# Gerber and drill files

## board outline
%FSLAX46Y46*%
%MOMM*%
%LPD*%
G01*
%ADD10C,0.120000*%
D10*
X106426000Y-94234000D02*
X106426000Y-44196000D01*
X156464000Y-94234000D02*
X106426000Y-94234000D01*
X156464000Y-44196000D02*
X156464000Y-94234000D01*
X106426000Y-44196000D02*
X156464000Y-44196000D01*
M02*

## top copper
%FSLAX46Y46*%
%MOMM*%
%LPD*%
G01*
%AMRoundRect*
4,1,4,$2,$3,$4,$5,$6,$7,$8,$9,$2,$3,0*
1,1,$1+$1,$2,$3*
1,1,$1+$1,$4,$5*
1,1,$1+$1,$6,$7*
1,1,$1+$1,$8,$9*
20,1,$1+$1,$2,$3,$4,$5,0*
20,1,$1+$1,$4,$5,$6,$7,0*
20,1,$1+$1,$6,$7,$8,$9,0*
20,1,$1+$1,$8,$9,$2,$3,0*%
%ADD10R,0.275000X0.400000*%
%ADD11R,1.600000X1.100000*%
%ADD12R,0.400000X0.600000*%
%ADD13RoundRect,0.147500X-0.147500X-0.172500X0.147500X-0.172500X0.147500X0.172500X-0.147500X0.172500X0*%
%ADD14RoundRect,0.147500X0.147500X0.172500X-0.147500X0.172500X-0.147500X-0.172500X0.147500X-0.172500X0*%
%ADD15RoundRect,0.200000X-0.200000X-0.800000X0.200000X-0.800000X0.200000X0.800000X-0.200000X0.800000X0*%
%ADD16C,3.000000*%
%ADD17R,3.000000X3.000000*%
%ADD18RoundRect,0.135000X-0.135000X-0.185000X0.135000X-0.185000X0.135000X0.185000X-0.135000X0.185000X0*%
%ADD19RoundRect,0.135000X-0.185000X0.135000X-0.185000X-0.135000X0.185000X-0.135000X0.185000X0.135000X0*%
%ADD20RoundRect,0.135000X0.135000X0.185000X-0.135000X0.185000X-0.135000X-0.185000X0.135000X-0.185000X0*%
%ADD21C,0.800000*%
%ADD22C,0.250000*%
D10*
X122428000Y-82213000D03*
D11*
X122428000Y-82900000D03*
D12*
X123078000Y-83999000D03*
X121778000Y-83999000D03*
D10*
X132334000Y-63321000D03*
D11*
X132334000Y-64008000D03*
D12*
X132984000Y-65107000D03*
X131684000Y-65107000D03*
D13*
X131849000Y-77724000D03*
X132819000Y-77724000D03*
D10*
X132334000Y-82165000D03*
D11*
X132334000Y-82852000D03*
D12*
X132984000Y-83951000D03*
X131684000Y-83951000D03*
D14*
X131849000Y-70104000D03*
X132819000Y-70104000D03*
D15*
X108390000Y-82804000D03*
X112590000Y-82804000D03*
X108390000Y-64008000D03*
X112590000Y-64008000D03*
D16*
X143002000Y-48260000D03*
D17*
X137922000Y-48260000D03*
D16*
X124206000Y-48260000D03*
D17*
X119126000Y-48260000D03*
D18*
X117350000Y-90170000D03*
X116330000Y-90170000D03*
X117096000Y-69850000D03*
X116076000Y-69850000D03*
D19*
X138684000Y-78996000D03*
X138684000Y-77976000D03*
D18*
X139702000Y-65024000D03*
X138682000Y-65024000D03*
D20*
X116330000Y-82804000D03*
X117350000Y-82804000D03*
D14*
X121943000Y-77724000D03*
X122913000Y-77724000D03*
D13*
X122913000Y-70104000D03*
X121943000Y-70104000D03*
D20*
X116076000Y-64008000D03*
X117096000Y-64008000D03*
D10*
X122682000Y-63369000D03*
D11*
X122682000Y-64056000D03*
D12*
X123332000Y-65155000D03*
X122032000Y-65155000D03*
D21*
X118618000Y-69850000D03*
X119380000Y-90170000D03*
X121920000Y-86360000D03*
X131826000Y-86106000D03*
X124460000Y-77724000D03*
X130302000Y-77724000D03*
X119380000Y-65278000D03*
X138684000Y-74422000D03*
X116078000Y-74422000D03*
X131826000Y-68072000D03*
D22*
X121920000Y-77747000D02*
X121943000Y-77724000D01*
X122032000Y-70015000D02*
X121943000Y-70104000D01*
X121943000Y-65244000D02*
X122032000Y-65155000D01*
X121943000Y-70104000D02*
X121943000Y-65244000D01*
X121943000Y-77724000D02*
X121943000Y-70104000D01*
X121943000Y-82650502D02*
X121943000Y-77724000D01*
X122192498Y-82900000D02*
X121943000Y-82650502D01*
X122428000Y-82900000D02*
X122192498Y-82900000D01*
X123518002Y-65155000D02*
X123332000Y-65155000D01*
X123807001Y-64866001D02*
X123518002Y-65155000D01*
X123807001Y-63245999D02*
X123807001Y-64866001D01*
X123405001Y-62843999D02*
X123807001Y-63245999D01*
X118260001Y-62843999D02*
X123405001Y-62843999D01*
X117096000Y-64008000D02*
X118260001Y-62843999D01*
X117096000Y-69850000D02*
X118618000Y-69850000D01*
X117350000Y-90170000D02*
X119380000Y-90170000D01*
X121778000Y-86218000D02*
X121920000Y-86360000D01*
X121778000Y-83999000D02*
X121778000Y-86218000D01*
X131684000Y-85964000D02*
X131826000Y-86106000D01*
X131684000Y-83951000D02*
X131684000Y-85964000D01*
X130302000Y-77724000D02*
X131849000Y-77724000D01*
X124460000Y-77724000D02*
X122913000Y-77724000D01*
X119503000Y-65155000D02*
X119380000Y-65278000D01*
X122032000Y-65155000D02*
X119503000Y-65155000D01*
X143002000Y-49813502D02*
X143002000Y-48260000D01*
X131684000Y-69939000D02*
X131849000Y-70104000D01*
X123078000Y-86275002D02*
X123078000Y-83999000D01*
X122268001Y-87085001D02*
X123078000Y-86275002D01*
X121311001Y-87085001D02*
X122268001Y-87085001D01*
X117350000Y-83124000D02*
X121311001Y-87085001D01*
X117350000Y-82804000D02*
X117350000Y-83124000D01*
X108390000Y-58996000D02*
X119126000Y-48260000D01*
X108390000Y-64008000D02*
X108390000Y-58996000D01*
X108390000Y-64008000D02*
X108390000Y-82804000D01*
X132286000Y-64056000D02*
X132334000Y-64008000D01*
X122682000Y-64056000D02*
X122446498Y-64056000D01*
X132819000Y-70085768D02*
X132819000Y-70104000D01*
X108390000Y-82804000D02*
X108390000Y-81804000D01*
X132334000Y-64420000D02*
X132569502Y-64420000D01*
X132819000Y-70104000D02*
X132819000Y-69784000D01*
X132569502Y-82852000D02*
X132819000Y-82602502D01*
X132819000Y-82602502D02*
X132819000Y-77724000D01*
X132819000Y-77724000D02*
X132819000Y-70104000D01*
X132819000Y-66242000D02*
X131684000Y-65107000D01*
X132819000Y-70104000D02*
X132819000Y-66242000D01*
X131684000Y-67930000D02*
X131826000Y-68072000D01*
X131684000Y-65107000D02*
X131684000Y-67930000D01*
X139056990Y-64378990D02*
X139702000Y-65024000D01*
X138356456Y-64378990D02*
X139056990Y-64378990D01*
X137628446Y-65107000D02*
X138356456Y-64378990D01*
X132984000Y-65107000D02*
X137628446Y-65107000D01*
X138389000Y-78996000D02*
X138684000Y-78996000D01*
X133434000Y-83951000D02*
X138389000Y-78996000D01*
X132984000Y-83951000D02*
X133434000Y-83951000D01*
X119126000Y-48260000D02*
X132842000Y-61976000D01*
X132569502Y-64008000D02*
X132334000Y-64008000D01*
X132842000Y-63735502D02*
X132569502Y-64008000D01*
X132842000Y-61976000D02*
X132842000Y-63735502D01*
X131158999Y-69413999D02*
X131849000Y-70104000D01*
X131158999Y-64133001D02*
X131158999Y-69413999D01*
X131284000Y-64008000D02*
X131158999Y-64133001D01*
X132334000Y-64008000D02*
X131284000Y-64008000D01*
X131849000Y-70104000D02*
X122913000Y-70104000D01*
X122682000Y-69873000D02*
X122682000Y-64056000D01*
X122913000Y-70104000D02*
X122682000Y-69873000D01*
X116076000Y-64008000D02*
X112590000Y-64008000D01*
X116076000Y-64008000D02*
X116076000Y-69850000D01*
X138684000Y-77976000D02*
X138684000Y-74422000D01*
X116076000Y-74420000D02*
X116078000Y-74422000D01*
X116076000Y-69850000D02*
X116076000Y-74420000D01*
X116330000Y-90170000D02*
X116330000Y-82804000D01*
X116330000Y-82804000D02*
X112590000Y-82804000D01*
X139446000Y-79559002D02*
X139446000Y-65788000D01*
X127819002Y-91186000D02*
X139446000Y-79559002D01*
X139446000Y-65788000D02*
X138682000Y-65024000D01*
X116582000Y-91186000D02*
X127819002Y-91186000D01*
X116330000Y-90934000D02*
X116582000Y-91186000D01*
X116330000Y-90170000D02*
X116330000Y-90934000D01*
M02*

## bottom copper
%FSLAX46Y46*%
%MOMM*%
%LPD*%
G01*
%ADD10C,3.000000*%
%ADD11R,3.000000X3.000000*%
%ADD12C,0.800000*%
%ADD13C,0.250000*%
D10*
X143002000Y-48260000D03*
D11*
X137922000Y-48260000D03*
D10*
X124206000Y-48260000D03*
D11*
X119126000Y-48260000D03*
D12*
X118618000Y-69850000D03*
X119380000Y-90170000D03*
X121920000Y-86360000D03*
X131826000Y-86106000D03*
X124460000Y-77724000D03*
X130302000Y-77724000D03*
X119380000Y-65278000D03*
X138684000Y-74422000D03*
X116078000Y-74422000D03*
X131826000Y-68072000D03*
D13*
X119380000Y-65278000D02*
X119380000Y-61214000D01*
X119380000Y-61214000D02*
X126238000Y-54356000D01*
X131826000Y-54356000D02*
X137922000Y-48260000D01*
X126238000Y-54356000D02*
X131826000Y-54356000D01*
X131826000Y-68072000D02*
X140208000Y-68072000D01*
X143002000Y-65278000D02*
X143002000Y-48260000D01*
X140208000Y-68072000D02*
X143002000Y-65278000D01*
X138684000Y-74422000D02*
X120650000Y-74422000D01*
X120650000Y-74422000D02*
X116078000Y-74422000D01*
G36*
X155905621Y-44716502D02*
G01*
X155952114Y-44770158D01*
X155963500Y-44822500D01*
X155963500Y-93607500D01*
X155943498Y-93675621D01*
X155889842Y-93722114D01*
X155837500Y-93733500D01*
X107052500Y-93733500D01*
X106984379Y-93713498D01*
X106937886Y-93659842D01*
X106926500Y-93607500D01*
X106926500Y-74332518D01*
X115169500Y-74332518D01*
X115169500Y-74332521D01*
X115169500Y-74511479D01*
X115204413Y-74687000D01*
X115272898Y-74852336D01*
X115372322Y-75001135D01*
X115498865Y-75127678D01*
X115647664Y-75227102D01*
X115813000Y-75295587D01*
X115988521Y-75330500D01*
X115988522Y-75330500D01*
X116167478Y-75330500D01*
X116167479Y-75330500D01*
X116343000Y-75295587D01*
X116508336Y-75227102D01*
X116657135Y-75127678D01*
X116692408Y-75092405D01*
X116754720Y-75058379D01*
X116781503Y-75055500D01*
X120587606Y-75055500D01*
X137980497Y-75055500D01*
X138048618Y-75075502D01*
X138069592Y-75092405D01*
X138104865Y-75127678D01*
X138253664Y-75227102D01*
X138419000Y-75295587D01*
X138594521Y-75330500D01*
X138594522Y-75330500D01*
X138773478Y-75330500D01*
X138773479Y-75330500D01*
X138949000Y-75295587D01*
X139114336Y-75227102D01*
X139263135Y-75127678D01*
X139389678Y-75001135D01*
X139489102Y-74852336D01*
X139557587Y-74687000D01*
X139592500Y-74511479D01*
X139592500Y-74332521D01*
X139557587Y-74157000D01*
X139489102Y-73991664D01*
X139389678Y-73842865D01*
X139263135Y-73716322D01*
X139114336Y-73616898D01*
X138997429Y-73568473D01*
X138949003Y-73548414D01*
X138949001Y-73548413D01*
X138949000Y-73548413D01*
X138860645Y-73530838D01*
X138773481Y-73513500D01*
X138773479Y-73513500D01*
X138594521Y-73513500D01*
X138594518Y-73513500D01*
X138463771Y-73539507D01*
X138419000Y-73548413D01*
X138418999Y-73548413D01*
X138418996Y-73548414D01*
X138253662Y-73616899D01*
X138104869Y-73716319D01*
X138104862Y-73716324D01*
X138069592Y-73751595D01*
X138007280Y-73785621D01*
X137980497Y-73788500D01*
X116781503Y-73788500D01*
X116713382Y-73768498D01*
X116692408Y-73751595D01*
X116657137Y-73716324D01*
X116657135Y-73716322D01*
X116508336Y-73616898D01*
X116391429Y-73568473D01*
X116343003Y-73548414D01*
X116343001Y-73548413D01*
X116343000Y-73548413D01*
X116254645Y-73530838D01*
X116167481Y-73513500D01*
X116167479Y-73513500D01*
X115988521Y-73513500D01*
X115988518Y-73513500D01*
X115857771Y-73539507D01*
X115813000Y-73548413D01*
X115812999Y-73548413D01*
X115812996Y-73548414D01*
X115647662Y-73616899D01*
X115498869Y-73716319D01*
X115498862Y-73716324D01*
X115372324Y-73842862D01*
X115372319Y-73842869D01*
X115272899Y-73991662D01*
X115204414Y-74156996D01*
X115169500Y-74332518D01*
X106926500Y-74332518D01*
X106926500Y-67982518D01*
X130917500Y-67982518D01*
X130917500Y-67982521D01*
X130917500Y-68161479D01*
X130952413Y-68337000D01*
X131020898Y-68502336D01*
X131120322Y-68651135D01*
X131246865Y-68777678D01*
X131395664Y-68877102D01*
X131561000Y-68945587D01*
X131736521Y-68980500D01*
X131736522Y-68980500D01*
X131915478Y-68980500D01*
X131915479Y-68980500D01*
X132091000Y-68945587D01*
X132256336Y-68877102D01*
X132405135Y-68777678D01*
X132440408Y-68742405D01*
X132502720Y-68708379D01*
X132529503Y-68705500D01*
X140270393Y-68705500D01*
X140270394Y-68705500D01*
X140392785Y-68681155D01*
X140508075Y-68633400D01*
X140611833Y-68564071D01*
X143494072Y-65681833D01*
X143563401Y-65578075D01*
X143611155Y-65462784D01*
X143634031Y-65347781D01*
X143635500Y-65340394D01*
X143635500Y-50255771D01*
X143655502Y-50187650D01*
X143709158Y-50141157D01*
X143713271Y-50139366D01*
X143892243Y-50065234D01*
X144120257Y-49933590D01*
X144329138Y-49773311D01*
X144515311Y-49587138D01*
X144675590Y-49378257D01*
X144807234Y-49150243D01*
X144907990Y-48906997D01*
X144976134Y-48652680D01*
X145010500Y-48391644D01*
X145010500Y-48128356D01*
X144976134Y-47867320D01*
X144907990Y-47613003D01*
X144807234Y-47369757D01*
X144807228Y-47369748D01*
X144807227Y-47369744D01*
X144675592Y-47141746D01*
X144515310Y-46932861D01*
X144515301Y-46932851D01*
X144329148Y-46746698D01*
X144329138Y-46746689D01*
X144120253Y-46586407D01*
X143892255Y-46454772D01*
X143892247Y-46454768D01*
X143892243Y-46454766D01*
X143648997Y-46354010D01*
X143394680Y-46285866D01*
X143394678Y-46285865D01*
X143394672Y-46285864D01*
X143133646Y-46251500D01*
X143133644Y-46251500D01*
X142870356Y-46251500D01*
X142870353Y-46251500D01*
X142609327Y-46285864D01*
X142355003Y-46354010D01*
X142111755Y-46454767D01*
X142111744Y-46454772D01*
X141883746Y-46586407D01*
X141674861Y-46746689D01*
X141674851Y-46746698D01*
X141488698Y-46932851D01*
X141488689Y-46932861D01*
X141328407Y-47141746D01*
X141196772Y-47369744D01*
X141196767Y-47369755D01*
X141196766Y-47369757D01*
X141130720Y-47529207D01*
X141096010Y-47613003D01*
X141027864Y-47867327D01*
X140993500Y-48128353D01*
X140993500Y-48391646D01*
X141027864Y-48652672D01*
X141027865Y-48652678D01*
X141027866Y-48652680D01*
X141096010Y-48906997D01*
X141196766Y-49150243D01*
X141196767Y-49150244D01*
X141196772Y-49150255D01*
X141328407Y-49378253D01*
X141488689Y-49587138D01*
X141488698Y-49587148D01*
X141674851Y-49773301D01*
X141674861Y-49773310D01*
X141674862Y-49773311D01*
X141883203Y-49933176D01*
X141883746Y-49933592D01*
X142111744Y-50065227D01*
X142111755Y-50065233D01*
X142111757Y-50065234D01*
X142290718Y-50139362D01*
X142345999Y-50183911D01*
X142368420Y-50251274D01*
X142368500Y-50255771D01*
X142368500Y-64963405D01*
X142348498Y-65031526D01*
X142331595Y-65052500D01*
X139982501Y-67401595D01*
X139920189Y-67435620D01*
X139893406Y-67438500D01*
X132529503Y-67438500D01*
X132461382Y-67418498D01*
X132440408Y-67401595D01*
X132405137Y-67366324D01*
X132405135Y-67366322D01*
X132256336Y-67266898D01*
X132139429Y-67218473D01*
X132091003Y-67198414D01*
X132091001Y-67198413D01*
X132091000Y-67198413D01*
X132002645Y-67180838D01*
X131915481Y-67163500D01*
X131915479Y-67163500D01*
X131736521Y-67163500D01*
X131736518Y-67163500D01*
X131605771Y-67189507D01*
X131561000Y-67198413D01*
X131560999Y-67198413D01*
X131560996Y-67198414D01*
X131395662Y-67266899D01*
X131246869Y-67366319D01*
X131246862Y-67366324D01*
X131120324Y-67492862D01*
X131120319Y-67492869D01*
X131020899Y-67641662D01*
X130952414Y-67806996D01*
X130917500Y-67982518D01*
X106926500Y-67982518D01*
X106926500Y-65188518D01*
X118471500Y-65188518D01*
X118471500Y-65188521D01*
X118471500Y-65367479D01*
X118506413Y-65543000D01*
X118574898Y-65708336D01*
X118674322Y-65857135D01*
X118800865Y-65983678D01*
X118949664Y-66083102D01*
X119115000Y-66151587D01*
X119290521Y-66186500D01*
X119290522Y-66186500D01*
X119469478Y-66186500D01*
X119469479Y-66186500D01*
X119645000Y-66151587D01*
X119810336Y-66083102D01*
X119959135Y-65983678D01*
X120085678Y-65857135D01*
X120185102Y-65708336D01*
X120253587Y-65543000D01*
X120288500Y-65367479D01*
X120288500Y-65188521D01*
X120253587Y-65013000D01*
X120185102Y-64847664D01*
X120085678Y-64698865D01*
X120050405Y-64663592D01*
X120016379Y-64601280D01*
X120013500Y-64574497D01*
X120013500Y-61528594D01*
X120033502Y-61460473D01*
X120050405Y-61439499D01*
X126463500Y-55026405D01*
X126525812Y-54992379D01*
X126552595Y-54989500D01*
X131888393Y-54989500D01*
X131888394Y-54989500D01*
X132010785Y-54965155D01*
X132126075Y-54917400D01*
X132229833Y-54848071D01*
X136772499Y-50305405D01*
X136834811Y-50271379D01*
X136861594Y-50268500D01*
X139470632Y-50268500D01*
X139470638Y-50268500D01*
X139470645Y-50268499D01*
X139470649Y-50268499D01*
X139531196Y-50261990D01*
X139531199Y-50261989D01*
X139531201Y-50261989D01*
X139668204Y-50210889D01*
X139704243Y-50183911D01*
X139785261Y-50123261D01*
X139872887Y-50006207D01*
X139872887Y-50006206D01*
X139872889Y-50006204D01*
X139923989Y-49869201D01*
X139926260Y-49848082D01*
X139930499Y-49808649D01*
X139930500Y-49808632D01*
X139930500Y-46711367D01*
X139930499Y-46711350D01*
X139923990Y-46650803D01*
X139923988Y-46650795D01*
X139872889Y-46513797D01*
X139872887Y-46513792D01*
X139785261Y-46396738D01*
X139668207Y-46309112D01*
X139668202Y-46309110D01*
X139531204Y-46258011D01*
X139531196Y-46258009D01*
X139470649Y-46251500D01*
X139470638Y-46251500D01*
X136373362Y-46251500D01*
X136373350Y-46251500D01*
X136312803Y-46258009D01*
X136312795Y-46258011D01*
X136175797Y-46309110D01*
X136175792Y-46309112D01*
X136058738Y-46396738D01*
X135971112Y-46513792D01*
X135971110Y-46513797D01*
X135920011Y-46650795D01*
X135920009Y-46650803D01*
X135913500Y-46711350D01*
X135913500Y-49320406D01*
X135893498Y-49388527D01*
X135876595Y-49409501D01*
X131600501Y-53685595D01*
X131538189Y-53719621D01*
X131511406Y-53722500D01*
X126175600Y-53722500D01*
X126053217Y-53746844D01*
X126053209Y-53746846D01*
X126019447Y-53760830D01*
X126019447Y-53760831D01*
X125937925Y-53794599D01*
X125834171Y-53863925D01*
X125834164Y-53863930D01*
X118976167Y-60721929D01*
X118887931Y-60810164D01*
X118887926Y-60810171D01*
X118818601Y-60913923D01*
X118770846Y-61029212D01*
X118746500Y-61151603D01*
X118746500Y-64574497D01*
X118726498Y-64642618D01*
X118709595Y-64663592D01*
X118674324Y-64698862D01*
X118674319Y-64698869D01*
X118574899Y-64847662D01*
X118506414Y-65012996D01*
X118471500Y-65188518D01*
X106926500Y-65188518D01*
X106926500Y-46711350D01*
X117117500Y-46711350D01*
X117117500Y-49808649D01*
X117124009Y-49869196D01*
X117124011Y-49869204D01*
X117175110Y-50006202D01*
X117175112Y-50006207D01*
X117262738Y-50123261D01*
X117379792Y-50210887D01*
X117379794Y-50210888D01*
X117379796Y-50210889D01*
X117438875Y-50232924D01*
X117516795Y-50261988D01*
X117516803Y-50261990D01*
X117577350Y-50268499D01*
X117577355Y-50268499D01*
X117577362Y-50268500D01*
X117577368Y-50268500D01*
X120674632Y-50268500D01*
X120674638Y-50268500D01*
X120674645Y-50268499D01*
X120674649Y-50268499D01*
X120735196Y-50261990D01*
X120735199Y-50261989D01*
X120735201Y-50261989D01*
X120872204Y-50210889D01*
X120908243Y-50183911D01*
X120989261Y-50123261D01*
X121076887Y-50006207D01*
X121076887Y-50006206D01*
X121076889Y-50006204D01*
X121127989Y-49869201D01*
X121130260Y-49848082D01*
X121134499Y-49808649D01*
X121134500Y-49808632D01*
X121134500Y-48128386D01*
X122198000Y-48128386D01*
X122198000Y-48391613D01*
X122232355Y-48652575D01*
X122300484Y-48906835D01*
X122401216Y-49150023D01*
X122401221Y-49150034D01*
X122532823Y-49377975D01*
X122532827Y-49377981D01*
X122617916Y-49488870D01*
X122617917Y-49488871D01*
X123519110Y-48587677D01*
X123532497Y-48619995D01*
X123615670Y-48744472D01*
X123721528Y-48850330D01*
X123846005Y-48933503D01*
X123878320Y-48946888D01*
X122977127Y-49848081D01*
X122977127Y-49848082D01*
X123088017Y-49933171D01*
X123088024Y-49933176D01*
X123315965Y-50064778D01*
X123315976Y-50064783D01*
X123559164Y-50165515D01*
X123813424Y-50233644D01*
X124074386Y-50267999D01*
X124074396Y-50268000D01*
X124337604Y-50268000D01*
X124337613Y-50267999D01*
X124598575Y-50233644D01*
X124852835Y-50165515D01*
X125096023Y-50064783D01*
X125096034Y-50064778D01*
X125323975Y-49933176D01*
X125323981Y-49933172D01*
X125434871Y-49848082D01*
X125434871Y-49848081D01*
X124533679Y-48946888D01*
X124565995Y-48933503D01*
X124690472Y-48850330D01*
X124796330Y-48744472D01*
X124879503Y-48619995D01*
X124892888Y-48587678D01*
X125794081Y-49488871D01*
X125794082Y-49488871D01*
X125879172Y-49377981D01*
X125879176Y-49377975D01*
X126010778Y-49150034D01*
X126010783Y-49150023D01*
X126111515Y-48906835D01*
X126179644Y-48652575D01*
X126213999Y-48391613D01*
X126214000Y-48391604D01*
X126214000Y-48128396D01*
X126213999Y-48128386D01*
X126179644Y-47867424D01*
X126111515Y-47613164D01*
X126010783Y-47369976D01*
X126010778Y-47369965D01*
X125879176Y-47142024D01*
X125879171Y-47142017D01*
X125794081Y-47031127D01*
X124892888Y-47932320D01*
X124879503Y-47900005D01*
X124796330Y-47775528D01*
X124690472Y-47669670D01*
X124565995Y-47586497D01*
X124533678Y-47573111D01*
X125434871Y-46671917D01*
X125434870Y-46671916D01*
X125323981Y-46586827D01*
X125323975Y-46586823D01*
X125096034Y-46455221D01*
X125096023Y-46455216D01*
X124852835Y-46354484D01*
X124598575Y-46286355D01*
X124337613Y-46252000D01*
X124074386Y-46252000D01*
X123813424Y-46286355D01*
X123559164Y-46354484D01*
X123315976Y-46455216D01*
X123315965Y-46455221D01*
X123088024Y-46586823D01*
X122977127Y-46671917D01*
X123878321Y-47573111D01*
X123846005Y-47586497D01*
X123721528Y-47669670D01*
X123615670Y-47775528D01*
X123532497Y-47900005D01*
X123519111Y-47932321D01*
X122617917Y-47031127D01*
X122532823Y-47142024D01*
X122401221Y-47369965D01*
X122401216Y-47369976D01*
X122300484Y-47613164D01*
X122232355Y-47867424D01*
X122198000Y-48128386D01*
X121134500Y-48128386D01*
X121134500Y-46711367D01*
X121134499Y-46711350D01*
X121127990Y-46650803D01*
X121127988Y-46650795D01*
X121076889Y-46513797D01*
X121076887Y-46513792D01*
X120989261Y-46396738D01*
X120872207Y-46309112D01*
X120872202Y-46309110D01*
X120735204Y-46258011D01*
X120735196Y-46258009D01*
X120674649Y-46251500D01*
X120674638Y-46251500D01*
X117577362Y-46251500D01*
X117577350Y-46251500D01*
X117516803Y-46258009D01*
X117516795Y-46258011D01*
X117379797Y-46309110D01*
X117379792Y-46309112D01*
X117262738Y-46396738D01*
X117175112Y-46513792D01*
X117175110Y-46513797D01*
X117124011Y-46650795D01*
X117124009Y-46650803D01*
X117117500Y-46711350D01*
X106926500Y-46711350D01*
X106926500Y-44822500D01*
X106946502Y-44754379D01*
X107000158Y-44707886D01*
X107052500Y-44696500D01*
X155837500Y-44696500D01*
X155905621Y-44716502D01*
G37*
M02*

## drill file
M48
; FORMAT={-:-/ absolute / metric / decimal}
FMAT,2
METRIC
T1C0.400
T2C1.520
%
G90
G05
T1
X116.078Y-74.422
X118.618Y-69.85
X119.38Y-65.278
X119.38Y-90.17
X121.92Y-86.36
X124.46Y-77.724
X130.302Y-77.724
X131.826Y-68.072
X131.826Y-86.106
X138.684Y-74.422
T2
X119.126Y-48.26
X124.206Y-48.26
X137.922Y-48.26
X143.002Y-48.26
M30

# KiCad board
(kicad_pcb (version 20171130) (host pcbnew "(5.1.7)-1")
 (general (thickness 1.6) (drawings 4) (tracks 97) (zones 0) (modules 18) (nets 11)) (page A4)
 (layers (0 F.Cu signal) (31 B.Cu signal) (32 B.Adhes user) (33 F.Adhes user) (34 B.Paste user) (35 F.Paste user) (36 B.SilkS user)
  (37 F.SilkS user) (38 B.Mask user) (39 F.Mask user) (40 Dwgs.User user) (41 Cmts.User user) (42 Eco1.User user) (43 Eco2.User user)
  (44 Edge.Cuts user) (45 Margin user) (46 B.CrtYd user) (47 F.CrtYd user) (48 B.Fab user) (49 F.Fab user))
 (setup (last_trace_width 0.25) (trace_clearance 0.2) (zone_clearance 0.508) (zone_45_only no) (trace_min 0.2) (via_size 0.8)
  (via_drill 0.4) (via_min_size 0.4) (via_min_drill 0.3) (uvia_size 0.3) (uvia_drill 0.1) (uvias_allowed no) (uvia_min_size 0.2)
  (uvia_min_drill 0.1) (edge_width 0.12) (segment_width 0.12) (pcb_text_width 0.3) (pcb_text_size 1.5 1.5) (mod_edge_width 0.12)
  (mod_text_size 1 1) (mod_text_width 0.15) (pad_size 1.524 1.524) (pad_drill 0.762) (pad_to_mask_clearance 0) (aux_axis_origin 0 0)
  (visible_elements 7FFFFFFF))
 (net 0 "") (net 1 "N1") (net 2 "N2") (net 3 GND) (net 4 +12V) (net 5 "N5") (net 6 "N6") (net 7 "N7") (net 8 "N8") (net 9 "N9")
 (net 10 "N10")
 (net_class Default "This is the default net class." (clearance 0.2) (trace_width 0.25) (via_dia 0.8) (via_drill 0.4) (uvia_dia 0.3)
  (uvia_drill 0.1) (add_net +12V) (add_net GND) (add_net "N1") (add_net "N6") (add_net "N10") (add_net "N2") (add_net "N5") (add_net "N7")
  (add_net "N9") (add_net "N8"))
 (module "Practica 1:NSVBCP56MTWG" (layer F.Cu) (at 122.428 83.106)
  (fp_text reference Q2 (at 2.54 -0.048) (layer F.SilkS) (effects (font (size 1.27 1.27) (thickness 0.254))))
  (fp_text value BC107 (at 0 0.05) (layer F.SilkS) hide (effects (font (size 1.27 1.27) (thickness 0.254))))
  (pad 4 smd rect (at 0 -0.893) (size 0.275 0.4) (layers F.Cu F.Paste F.Mask))
  (pad 3 smd rect (at 0 -0.206 90) (size 1.1 1.6) (layers F.Cu F.Paste F.Mask) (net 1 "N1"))
  (pad 2 smd rect (at 0.65 0.893) (size 0.4 0.6) (layers F.Cu F.Paste F.Mask) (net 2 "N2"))
  (pad 1 smd rect (at -0.65 0.893) (size 0.4 0.6) (layers F.Cu F.Paste F.Mask) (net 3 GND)))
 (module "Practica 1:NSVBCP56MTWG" (layer F.Cu) (at 132.334 64.214)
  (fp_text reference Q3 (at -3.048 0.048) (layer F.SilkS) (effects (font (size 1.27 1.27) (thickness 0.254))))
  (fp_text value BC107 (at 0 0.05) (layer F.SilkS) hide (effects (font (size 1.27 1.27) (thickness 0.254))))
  (pad 4 smd rect (at 0 -0.893) (size 0.275 0.4) (layers F.Cu F.Paste F.Mask))
  (pad 3 smd rect (at 0 -0.206 90) (size 1.1 1.6) (layers F.Cu F.Paste F.Mask) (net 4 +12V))
  (pad 2 smd rect (at 0.65 0.893) (size 0.4 0.6) (layers F.Cu F.Paste F.Mask) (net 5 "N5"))
  (pad 1 smd rect (at -0.65 0.893) (size 0.4 0.6) (layers F.Cu F.Paste F.Mask) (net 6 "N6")))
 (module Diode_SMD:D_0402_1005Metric (layer F.Cu) (at 132.334 77.724)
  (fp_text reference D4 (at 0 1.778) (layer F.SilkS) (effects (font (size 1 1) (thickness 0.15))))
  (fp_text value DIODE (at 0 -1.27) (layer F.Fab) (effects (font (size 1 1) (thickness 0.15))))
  (pad 1 smd roundrect (at -0.485 0) (size 0.59 0.64) (layers F.Cu F.Paste F.Mask) (roundrect_rratio 0.25) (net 3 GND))
  (pad 2 smd roundrect (at 0.485 0) (size 0.59 0.64) (layers F.Cu F.Paste F.Mask) (roundrect_rratio 0.25) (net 6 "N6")))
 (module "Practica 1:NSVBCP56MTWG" (layer F.Cu) (at 132.334 83.058)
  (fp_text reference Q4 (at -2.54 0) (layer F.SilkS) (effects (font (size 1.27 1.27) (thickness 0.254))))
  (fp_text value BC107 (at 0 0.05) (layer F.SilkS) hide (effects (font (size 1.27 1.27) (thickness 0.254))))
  (pad 4 smd rect (at 0 -0.893) (size 0.275 0.4) (layers F.Cu F.Paste F.Mask))
  (pad 3 smd rect (at 0 -0.206 90) (size 1.1 1.6) (layers F.Cu F.Paste F.Mask) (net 6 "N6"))
  (pad 2 smd rect (at 0.65 0.893) (size 0.4 0.6) (layers F.Cu F.Paste F.Mask) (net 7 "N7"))
  (pad 1 smd rect (at -0.65 0.893) (size 0.4 0.6) (layers F.Cu F.Paste F.Mask) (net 3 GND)))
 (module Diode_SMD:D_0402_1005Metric (layer F.Cu) (at 132.334 70.104 180)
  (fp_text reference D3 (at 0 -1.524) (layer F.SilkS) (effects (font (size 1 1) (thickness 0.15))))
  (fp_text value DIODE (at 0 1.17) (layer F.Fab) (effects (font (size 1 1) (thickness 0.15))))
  (pad 2 smd roundrect (at 0.485 0 180) (size 0.59 0.64) (layers F.Cu F.Paste F.Mask) (roundrect_rratio 0.25) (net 4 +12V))
  (pad 1 smd roundrect (at -0.485 0 180) (size 0.59 0.64) (layers F.Cu F.Paste F.Mask) (roundrect_rratio 0.25) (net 6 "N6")))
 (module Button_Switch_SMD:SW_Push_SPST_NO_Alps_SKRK (layer F.Cu) (at 110.49 82.804)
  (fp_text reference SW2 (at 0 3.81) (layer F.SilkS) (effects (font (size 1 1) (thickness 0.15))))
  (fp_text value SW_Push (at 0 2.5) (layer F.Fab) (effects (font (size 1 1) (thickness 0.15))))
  (pad 1 smd roundrect (at -2.1 0) (size 0.8 2) (layers F.Cu F.Paste F.Mask) (roundrect_rratio 0.25) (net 4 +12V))
  (pad 2 smd roundrect (at 2.1 0) (size 0.8 2) (layers F.Cu F.Paste F.Mask) (roundrect_rratio 0.25) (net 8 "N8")))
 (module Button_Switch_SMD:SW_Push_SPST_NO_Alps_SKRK (layer F.Cu) (at 110.49 64.008)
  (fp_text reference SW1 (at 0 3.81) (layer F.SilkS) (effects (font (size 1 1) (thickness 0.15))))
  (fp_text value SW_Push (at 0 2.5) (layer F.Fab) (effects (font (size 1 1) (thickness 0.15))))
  (pad 1 smd roundrect (at -2.1 0) (size 0.8 2) (layers F.Cu F.Paste F.Mask) (roundrect_rratio 0.25) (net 4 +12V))
  (pad 2 smd roundrect (at 2.1 0) (size 0.8 2) (layers F.Cu F.Paste F.Mask) (roundrect_rratio 0.25) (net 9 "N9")))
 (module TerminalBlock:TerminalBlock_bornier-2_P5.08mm (layer F.Cu) (at 137.922 48.26)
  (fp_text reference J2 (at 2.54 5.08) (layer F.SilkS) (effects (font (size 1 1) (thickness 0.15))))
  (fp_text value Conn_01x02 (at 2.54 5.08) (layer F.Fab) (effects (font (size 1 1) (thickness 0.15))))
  (pad 2 thru_hole circle (at 5.08 0) (size 3 3) (drill 1.52) (layers *.Cu *.Mask) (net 6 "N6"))
  (pad 1 thru_hole rect (at 0 0) (size 3 3) (drill 1.52) (layers *.Cu *.Mask) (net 1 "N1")))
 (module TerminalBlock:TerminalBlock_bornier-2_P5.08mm (layer F.Cu) (at 119.126 48.26)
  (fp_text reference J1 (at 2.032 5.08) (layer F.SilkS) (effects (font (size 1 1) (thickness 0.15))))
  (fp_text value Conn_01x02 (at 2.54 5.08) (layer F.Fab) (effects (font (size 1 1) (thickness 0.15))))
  (pad 2 thru_hole circle (at 5.08 0) (size 3 3) (drill 1.52) (layers *.Cu *.Mask) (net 3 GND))
  (pad 1 thru_hole rect (at 0 0) (size 3 3) (drill 1.52) (layers *.Cu *.Mask) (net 4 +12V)))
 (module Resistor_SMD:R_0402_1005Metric (layer F.Cu) (at 116.84 90.17)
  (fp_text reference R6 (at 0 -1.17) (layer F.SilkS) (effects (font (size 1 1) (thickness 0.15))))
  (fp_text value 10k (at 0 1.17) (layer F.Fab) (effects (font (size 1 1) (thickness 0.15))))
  (pad 2 smd roundrect (at 0.51 0) (size 0.54 0.64) (layers F.Cu F.Paste F.Mask) (roundrect_rratio 0.25) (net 3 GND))
  (pad 1 smd roundrect (at -0.51 0) (size 0.54 0.64) (layers F.Cu F.Paste F.Mask) (roundrect_rratio 0.25) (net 8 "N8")))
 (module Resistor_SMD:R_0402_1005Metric (layer F.Cu) (at 116.586 69.85)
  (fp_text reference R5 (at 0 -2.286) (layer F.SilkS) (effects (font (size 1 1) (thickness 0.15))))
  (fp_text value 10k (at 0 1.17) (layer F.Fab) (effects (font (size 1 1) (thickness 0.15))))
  (pad 2 smd roundrect (at 0.51 0) (size 0.54 0.64) (layers F.Cu F.Paste F.Mask) (roundrect_rratio 0.25) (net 3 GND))
  (pad 1 smd roundrect (at -0.51 0) (size 0.54 0.64) (layers F.Cu F.Paste F.Mask) (roundrect_rratio 0.25) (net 9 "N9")))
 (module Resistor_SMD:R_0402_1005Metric (layer F.Cu) (at 138.684 78.486 270)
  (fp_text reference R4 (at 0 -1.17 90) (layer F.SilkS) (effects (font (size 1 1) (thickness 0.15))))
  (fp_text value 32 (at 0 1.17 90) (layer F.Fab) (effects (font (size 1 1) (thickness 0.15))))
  (pad 2 smd roundrect (at 0.51 0 270) (size 0.54 0.64) (layers F.Cu F.Paste F.Mask) (roundrect_rratio 0.25) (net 7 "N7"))
  (pad 1 smd roundrect (at -0.51 0 270) (size 0.54 0.64) (layers F.Cu F.Paste F.Mask) (roundrect_rratio 0.25) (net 9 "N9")))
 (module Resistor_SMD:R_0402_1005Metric (layer F.Cu) (at 139.192 65.024)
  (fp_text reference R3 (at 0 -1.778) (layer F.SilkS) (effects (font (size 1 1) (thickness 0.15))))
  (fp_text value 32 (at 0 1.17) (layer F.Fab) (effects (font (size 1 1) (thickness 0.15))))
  (pad 2 smd roundrect (at 0.51 0) (size 0.54 0.64) (layers F.Cu F.Paste F.Mask) (roundrect_rratio 0.25) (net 5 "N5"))
  (pad 1 smd roundrect (at -0.51 0) (size 0.54 0.64) (layers F.Cu F.Paste F.Mask) (roundrect_rratio 0.25) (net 8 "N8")))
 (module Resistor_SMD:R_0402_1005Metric (layer F.Cu) (at 116.84 82.804 180)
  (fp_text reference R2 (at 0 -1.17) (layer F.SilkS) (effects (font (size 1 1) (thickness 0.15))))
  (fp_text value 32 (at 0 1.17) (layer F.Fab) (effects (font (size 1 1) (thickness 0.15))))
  (pad 2 smd roundrect (at 0.51 0 180) (size 0.54 0.64) (layers F.Cu F.Paste F.Mask) (roundrect_rratio 0.25) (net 8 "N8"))
  (pad 1 smd roundrect (at -0.51 0 180) (size 0.54 0.64) (layers F.Cu F.Paste F.Mask) (roundrect_rratio 0.25) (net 2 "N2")))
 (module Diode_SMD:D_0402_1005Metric (layer F.Cu) (at 122.428 77.724 180)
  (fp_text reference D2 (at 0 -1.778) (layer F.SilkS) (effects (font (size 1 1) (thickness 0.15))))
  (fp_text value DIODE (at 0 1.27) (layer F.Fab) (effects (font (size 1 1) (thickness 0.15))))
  (pad 2 smd roundrect (at 0.485 0 180) (size 0.59 0.64) (layers F.Cu F.Paste F.Mask) (roundrect_rratio 0.25) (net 1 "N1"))
  (pad 1 smd roundrect (at -0.485 0 180) (size 0.59 0.64) (layers F.Cu F.Paste F.Mask) (roundrect_rratio 0.25) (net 3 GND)))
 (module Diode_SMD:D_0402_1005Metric (layer F.Cu) (at 122.428 70.104)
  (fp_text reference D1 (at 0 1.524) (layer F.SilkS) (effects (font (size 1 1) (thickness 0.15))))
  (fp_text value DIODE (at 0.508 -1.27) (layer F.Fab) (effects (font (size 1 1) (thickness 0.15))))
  (pad 2 smd roundrect (at 0.485 0) (size 0.59 0.64) (layers F.Cu F.Paste F.Mask) (roundrect_rratio 0.25) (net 4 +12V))
  (pad 1 smd roundrect (at -0.485 0) (size 0.59 0.64) (layers F.Cu F.Paste F.Mask) (roundrect_rratio 0.25) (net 1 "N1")))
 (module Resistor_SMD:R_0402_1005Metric (layer F.Cu) (at 116.586 64.008 180)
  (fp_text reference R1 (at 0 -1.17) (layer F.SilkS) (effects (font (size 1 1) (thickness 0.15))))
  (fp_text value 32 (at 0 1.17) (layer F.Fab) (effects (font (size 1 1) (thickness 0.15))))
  (pad 2 smd roundrect (at 0.51 0 180) (size 0.54 0.64) (layers F.Cu F.Paste F.Mask) (roundrect_rratio 0.25) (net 9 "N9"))
  (pad 1 smd roundrect (at -0.51 0 180) (size 0.54 0.64) (layers F.Cu F.Paste F.Mask) (roundrect_rratio 0.25) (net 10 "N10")))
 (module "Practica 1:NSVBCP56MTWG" (layer F.Cu) (at 122.682 64.262)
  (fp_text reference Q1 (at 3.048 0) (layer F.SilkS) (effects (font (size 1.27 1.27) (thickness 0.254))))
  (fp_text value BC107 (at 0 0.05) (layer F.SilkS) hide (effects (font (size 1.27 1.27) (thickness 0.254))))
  (pad 4 smd rect (at 0 -0.893) (size 0.275 0.4) (layers F.Cu F.Paste F.Mask))
  (pad 3 smd rect (at 0 -0.206 90) (size 1.1 1.6) (layers F.Cu F.Paste F.Mask) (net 4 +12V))
  (pad 2 smd rect (at 0.65 0.893) (size 0.4 0.6) (layers F.Cu F.Paste F.Mask) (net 10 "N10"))
  (pad 1 smd rect (at -0.65 0.893) (size 0.4 0.6) (layers F.Cu F.Paste F.Mask) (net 1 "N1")))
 (gr_line (start 106.426 94.234) (end 106.426 44.196) (layer Edge.Cuts) (width 0.12))
 (gr_line (start 156.464 94.234) (end 106.426 94.234) (layer Edge.Cuts) (width 0.12))
 (gr_line (start 156.464 44.196) (end 156.464 94.234) (layer Edge.Cuts) (width 0.12))
 (gr_line (start 106.426 44.196) (end 156.464 44.196) (layer Edge.Cuts) (width 0.12))
 (via (at 118.618 69.85) (size 0.8) (drill 0.4) (layers F.Cu B.Cu) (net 3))
 (segment (start 121.92 77.747) (end 121.943 77.724) (width 0.25) (layer F.Cu) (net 1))
 (segment (start 122.032 70.015) (end 121.943 70.104) (width 0.25) (layer F.Cu) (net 1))
 (segment (start 121.943 65.244) (end 122.032 65.155) (width 0.25) (layer F.Cu) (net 1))
 (segment (start 121.943 70.104) (end 121.943 65.244) (width 0.25) (layer F.Cu) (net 1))
 (segment (start 121.943 77.724) (end 121.943 70.104) (width 0.25) (layer F.Cu) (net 1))
 (segment (start 121.943 82.650502) (end 121.943 77.724) (width 0.25) (layer F.Cu) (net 1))
 (segment (start 122.192498 82.9) (end 121.943 82.650502) (width 0.25) (layer F.Cu) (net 1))
 (segment (start 122.428 82.9) (end 122.192498 82.9) (width 0.25) (layer F.Cu) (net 1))
 (segment (start 123.518002 65.155) (end 123.332 65.155) (width 0.25) (layer F.Cu) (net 10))
 (segment (start 123.807001 64.866001) (end 123.518002 65.155) (width 0.25) (layer F.Cu) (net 10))
 (segment (start 123.807001 63.245999) (end 123.807001 64.866001) (width 0.25) (layer F.Cu) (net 10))
 (segment (start 123.405001 62.843999) (end 123.807001 63.245999) (width 0.25) (layer F.Cu) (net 10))
 (segment (start 118.260001 62.843999) (end 123.405001 62.843999) (width 0.25) (layer F.Cu) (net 10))
 (segment (start 117.096 64.008) (end 118.260001 62.843999) (width 0.25) (layer F.Cu) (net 10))
 (segment (start 117.096 69.85) (end 118.618 69.85) (width 0.25) (layer F.Cu) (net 3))
 (via (at 119.38 90.17) (size 0.8) (drill 0.4) (layers F.Cu B.Cu) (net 3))
 (segment (start 117.35 90.17) (end 119.38 90.17) (width 0.25) (layer F.Cu) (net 3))
 (via (at 121.92 86.36) (size 0.8) (drill 0.4) (layers F.Cu B.Cu) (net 3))
 (segment (start 121.778 86.218) (end 121.92 86.36) (width 0.25) (layer F.Cu) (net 3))
 (segment (start 121.778 83.999) (end 121.778 86.218) (width 0.25) (layer F.Cu) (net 3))
 (via (at 131.826 86.106) (size 0.8) (drill 0.4) (layers F.Cu B.Cu) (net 3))
 (segment (start 131.684 85.964) (end 131.826 86.106) (width 0.25) (layer F.Cu) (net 3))
 (segment (start 131.684 83.951) (end 131.684 85.964) (width 0.25) (layer F.Cu) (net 3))
 (via (at 124.46 77.724) (size 0.8) (drill 0.4) (layers F.Cu B.Cu) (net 3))
 (via (at 130.302 77.724) (size 0.8) (drill 0.4) (layers F.Cu B.Cu) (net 3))
 (segment (start 130.302 77.724) (end 131.849 77.724) (width 0.25) (layer F.Cu) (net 3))
 (segment (start 124.46 77.724) (end 122.913 77.724) (width 0.25) (layer F.Cu) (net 3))
 (via (at 119.38 65.278) (size 0.8) (drill 0.4) (layers F.Cu B.Cu) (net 1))
 (segment (start 119.503 65.155) (end 119.38 65.278) (width 0.25) (layer F.Cu) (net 1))
 (segment (start 122.032 65.155) (end 119.503 65.155) (width 0.25) (layer F.Cu) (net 1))
 (segment (start 119.38 65.278) (end 119.38 61.214) (width 0.25) (layer B.Cu) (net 1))
 (segment (start 119.38 61.214) (end 126.238 54.356) (width 0.25) (layer B.Cu) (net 1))
 (segment (start 131.826 54.356) (end 137.922 48.26) (width 0.25) (layer B.Cu) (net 1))
 (segment (start 126.238 54.356) (end 131.826 54.356) (width 0.25) (layer B.Cu) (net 1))
 (via (at 138.684 74.422) (size 0.8) (drill 0.4) (layers F.Cu B.Cu) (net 9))
 (via (at 116.078 74.422) (size 0.8) (drill 0.4) (layers F.Cu B.Cu) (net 9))
 (via (at 131.826 68.072) (size 0.8) (drill 0.4) (layers F.Cu B.Cu) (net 6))
 (segment (start 143.002 49.813502) (end 143.002 48.26) (width 0.25) (layer F.Cu) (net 6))
 (segment (start 131.684 69.939) (end 131.849 70.104) (width 0.25) (layer F.Cu) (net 4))
 (segment (start 123.078 86.275002) (end 123.078 83.999) (width 0.25) (layer F.Cu) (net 2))
 (segment (start 122.268001 87.085001) (end 123.078 86.275002) (width 0.25) (layer F.Cu) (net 2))
 (segment (start 121.311001 87.085001) (end 122.268001 87.085001) (width 0.25) (layer F.Cu) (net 2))
 (segment (start 117.35 83.124) (end 121.311001 87.085001) (width 0.25) (layer F.Cu) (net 2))
 (segment (start 117.35 82.804) (end 117.35 83.124) (width 0.25) (layer F.Cu) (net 2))
 (segment (start 108.39 58.996) (end 119.126 48.26) (width 0.25) (layer F.Cu) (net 4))
 (segment (start 108.39 64.008) (end 108.39 58.996) (width 0.25) (layer F.Cu) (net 4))
 (segment (start 108.39 64.008) (end 108.39 82.804) (width 0.25) (layer F.Cu) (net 4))
 (segment (start 132.286 64.056) (end 132.334 64.008) (width 0.25) (layer F.Cu) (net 4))
 (segment (start 122.682 64.056) (end 122.446498 64.056) (width 0.25) (layer F.Cu) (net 4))
 (segment (start 132.819 70.085768) (end 132.819 70.104) (width 0.25) (layer F.Cu) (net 6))
 (segment (start 108.39 82.804) (end 108.39 81.804) (width 0.25) (layer F.Cu) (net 4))
 (segment (start 132.334 64.42) (end 132.569502 64.42) (width 0.25) (layer F.Cu) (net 4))
 (segment (start 132.819 70.104) (end 132.819 69.784) (width 0.25) (layer F.Cu) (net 6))
 (segment (start 132.569502 82.852) (end 132.819 82.602502) (width 0.25) (layer F.Cu) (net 6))
 (segment (start 132.819 82.602502) (end 132.819 77.724) (width 0.25) (layer F.Cu) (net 6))
 (segment (start 132.819 77.724) (end 132.819 70.104) (width 0.25) (layer F.Cu) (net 6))
 (segment (start 132.819 66.242) (end 131.684 65.107) (width 0.25) (layer F.Cu) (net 6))
 (segment (start 132.819 70.104) (end 132.819 66.242) (width 0.25) (layer F.Cu) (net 6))
 (segment (start 131.684 67.93) (end 131.826 68.072) (width 0.25) (layer F.Cu) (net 6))
 (segment (start 131.684 65.107) (end 131.684 67.93) (width 0.25) (layer F.Cu) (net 6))
 (segment (start 131.826 68.072) (end 140.208 68.072) (width 0.25) (layer B.Cu) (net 6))
 (segment (start 143.002 65.278) (end 143.002 48.26) (width 0.25) (layer B.Cu) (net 6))
 (segment (start 140.208 68.072) (end 143.002 65.278) (width 0.25) (layer B.Cu) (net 6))
 (segment (start 139.05699 64.37899) (end 139.702 65.024) (width 0.25) (layer F.Cu) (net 5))
 (segment (start 138.356456 64.37899) (end 139.05699 64.37899) (width 0.25) (layer F.Cu) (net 5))
 (segment (start 137.628446 65.107) (end 138.356456 64.37899) (width 0.25) (layer F.Cu) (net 5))
 (segment (start 132.984 65.107) (end 137.628446 65.107) (width 0.25) (layer F.Cu) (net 5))
 (segment (start 138.389 78.996) (end 138.684 78.996) (width 0.25) (layer F.Cu) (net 7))
 (segment (start 133.434 83.951) (end 138.389 78.996) (width 0.25) (layer F.Cu) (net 7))
 (segment (start 132.984 83.951) (end 133.434 83.951) (width 0.25) (layer F.Cu) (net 7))
 (segment (start 119.126 48.26) (end 132.842 61.976) (width 0.25) (layer F.Cu) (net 4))
 (segment (start 132.569502 64.008) (end 132.334 64.008) (width 0.25) (layer F.Cu) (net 4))
 (segment (start 132.842 63.735502) (end 132.569502 64.008) (width 0.25) (layer F.Cu) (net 4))
 (segment (start 132.842 61.976) (end 132.842 63.735502) (width 0.25) (layer F.Cu) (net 4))
 (segment (start 131.158999 69.413999) (end 131.849 70.104) (width 0.25) (layer F.Cu) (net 4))
 (segment (start 131.158999 64.133001) (end 131.158999 69.413999) (width 0.25) (layer F.Cu) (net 4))
 (segment (start 131.284 64.008) (end 131.158999 64.133001) (width 0.25) (layer F.Cu) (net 4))
 (segment (start 132.334 64.008) (end 131.284 64.008) (width 0.25) (layer F.Cu) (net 4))
 (segment (start 131.849 70.104) (end 122.913 70.104) (width 0.25) (layer F.Cu) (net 4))
 (segment (start 122.682 69.873) (end 122.682 64.056) (width 0.25) (layer F.Cu) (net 4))
 (segment (start 122.913 70.104) (end 122.682 69.873) (width 0.25) (layer F.Cu) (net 4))
 (segment (start 116.076 64.008) (end 112.59 64.008) (width 0.25) (layer F.Cu) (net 9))
 (segment (start 116.076 64.008) (end 116.076 69.85) (width 0.25) (layer F.Cu) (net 9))
 (segment (start 138.684 77.976) (end 138.684 74.422) (width 0.25) (layer F.Cu) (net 9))
 (segment (start 138.684 74.422) (end 120.65 74.422) (width 0.25) (layer B.Cu) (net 9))
 (segment (start 120.65 74.422) (end 116.078 74.422) (width 0.25) (layer B.Cu) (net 9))
 (segment (start 116.076 74.42) (end 116.078 74.422) (width 0.25) (layer F.Cu) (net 9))
 (segment (start 116.076 69.85) (end 116.076 74.42) (width 0.25) (layer F.Cu) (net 9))
 (segment (start 116.33 90.17) (end 116.33 82.804) (width 0.25) (layer F.Cu) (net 8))
 (segment (start 116.33 82.804) (end 112.59 82.804) (width 0.25) (layer F.Cu) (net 8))
 (segment (start 139.446 79.559002) (end 139.446 65.788) (width 0.25) (layer F.Cu) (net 8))
 (segment (start 127.819002 91.186) (end 139.446 79.559002) (width 0.25) (layer F.Cu) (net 8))
 (segment (start 139.446 65.788) (end 138.682 65.024) (width 0.25) (layer F.Cu) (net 8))
 (segment (start 116.582 91.186) (end 127.819002 91.186) (width 0.25) (layer F.Cu) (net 8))
 (segment (start 116.33 90.934) (end 116.582 91.186) (width 0.25) (layer F.Cu) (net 8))
 (segment (start 116.33 90.17) (end 116.33 90.934) (width 0.25) (layer F.Cu) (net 8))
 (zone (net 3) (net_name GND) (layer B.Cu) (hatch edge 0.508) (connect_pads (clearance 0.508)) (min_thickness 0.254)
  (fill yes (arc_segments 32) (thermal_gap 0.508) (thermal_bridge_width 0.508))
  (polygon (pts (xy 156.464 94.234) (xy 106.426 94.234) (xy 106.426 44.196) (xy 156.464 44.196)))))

